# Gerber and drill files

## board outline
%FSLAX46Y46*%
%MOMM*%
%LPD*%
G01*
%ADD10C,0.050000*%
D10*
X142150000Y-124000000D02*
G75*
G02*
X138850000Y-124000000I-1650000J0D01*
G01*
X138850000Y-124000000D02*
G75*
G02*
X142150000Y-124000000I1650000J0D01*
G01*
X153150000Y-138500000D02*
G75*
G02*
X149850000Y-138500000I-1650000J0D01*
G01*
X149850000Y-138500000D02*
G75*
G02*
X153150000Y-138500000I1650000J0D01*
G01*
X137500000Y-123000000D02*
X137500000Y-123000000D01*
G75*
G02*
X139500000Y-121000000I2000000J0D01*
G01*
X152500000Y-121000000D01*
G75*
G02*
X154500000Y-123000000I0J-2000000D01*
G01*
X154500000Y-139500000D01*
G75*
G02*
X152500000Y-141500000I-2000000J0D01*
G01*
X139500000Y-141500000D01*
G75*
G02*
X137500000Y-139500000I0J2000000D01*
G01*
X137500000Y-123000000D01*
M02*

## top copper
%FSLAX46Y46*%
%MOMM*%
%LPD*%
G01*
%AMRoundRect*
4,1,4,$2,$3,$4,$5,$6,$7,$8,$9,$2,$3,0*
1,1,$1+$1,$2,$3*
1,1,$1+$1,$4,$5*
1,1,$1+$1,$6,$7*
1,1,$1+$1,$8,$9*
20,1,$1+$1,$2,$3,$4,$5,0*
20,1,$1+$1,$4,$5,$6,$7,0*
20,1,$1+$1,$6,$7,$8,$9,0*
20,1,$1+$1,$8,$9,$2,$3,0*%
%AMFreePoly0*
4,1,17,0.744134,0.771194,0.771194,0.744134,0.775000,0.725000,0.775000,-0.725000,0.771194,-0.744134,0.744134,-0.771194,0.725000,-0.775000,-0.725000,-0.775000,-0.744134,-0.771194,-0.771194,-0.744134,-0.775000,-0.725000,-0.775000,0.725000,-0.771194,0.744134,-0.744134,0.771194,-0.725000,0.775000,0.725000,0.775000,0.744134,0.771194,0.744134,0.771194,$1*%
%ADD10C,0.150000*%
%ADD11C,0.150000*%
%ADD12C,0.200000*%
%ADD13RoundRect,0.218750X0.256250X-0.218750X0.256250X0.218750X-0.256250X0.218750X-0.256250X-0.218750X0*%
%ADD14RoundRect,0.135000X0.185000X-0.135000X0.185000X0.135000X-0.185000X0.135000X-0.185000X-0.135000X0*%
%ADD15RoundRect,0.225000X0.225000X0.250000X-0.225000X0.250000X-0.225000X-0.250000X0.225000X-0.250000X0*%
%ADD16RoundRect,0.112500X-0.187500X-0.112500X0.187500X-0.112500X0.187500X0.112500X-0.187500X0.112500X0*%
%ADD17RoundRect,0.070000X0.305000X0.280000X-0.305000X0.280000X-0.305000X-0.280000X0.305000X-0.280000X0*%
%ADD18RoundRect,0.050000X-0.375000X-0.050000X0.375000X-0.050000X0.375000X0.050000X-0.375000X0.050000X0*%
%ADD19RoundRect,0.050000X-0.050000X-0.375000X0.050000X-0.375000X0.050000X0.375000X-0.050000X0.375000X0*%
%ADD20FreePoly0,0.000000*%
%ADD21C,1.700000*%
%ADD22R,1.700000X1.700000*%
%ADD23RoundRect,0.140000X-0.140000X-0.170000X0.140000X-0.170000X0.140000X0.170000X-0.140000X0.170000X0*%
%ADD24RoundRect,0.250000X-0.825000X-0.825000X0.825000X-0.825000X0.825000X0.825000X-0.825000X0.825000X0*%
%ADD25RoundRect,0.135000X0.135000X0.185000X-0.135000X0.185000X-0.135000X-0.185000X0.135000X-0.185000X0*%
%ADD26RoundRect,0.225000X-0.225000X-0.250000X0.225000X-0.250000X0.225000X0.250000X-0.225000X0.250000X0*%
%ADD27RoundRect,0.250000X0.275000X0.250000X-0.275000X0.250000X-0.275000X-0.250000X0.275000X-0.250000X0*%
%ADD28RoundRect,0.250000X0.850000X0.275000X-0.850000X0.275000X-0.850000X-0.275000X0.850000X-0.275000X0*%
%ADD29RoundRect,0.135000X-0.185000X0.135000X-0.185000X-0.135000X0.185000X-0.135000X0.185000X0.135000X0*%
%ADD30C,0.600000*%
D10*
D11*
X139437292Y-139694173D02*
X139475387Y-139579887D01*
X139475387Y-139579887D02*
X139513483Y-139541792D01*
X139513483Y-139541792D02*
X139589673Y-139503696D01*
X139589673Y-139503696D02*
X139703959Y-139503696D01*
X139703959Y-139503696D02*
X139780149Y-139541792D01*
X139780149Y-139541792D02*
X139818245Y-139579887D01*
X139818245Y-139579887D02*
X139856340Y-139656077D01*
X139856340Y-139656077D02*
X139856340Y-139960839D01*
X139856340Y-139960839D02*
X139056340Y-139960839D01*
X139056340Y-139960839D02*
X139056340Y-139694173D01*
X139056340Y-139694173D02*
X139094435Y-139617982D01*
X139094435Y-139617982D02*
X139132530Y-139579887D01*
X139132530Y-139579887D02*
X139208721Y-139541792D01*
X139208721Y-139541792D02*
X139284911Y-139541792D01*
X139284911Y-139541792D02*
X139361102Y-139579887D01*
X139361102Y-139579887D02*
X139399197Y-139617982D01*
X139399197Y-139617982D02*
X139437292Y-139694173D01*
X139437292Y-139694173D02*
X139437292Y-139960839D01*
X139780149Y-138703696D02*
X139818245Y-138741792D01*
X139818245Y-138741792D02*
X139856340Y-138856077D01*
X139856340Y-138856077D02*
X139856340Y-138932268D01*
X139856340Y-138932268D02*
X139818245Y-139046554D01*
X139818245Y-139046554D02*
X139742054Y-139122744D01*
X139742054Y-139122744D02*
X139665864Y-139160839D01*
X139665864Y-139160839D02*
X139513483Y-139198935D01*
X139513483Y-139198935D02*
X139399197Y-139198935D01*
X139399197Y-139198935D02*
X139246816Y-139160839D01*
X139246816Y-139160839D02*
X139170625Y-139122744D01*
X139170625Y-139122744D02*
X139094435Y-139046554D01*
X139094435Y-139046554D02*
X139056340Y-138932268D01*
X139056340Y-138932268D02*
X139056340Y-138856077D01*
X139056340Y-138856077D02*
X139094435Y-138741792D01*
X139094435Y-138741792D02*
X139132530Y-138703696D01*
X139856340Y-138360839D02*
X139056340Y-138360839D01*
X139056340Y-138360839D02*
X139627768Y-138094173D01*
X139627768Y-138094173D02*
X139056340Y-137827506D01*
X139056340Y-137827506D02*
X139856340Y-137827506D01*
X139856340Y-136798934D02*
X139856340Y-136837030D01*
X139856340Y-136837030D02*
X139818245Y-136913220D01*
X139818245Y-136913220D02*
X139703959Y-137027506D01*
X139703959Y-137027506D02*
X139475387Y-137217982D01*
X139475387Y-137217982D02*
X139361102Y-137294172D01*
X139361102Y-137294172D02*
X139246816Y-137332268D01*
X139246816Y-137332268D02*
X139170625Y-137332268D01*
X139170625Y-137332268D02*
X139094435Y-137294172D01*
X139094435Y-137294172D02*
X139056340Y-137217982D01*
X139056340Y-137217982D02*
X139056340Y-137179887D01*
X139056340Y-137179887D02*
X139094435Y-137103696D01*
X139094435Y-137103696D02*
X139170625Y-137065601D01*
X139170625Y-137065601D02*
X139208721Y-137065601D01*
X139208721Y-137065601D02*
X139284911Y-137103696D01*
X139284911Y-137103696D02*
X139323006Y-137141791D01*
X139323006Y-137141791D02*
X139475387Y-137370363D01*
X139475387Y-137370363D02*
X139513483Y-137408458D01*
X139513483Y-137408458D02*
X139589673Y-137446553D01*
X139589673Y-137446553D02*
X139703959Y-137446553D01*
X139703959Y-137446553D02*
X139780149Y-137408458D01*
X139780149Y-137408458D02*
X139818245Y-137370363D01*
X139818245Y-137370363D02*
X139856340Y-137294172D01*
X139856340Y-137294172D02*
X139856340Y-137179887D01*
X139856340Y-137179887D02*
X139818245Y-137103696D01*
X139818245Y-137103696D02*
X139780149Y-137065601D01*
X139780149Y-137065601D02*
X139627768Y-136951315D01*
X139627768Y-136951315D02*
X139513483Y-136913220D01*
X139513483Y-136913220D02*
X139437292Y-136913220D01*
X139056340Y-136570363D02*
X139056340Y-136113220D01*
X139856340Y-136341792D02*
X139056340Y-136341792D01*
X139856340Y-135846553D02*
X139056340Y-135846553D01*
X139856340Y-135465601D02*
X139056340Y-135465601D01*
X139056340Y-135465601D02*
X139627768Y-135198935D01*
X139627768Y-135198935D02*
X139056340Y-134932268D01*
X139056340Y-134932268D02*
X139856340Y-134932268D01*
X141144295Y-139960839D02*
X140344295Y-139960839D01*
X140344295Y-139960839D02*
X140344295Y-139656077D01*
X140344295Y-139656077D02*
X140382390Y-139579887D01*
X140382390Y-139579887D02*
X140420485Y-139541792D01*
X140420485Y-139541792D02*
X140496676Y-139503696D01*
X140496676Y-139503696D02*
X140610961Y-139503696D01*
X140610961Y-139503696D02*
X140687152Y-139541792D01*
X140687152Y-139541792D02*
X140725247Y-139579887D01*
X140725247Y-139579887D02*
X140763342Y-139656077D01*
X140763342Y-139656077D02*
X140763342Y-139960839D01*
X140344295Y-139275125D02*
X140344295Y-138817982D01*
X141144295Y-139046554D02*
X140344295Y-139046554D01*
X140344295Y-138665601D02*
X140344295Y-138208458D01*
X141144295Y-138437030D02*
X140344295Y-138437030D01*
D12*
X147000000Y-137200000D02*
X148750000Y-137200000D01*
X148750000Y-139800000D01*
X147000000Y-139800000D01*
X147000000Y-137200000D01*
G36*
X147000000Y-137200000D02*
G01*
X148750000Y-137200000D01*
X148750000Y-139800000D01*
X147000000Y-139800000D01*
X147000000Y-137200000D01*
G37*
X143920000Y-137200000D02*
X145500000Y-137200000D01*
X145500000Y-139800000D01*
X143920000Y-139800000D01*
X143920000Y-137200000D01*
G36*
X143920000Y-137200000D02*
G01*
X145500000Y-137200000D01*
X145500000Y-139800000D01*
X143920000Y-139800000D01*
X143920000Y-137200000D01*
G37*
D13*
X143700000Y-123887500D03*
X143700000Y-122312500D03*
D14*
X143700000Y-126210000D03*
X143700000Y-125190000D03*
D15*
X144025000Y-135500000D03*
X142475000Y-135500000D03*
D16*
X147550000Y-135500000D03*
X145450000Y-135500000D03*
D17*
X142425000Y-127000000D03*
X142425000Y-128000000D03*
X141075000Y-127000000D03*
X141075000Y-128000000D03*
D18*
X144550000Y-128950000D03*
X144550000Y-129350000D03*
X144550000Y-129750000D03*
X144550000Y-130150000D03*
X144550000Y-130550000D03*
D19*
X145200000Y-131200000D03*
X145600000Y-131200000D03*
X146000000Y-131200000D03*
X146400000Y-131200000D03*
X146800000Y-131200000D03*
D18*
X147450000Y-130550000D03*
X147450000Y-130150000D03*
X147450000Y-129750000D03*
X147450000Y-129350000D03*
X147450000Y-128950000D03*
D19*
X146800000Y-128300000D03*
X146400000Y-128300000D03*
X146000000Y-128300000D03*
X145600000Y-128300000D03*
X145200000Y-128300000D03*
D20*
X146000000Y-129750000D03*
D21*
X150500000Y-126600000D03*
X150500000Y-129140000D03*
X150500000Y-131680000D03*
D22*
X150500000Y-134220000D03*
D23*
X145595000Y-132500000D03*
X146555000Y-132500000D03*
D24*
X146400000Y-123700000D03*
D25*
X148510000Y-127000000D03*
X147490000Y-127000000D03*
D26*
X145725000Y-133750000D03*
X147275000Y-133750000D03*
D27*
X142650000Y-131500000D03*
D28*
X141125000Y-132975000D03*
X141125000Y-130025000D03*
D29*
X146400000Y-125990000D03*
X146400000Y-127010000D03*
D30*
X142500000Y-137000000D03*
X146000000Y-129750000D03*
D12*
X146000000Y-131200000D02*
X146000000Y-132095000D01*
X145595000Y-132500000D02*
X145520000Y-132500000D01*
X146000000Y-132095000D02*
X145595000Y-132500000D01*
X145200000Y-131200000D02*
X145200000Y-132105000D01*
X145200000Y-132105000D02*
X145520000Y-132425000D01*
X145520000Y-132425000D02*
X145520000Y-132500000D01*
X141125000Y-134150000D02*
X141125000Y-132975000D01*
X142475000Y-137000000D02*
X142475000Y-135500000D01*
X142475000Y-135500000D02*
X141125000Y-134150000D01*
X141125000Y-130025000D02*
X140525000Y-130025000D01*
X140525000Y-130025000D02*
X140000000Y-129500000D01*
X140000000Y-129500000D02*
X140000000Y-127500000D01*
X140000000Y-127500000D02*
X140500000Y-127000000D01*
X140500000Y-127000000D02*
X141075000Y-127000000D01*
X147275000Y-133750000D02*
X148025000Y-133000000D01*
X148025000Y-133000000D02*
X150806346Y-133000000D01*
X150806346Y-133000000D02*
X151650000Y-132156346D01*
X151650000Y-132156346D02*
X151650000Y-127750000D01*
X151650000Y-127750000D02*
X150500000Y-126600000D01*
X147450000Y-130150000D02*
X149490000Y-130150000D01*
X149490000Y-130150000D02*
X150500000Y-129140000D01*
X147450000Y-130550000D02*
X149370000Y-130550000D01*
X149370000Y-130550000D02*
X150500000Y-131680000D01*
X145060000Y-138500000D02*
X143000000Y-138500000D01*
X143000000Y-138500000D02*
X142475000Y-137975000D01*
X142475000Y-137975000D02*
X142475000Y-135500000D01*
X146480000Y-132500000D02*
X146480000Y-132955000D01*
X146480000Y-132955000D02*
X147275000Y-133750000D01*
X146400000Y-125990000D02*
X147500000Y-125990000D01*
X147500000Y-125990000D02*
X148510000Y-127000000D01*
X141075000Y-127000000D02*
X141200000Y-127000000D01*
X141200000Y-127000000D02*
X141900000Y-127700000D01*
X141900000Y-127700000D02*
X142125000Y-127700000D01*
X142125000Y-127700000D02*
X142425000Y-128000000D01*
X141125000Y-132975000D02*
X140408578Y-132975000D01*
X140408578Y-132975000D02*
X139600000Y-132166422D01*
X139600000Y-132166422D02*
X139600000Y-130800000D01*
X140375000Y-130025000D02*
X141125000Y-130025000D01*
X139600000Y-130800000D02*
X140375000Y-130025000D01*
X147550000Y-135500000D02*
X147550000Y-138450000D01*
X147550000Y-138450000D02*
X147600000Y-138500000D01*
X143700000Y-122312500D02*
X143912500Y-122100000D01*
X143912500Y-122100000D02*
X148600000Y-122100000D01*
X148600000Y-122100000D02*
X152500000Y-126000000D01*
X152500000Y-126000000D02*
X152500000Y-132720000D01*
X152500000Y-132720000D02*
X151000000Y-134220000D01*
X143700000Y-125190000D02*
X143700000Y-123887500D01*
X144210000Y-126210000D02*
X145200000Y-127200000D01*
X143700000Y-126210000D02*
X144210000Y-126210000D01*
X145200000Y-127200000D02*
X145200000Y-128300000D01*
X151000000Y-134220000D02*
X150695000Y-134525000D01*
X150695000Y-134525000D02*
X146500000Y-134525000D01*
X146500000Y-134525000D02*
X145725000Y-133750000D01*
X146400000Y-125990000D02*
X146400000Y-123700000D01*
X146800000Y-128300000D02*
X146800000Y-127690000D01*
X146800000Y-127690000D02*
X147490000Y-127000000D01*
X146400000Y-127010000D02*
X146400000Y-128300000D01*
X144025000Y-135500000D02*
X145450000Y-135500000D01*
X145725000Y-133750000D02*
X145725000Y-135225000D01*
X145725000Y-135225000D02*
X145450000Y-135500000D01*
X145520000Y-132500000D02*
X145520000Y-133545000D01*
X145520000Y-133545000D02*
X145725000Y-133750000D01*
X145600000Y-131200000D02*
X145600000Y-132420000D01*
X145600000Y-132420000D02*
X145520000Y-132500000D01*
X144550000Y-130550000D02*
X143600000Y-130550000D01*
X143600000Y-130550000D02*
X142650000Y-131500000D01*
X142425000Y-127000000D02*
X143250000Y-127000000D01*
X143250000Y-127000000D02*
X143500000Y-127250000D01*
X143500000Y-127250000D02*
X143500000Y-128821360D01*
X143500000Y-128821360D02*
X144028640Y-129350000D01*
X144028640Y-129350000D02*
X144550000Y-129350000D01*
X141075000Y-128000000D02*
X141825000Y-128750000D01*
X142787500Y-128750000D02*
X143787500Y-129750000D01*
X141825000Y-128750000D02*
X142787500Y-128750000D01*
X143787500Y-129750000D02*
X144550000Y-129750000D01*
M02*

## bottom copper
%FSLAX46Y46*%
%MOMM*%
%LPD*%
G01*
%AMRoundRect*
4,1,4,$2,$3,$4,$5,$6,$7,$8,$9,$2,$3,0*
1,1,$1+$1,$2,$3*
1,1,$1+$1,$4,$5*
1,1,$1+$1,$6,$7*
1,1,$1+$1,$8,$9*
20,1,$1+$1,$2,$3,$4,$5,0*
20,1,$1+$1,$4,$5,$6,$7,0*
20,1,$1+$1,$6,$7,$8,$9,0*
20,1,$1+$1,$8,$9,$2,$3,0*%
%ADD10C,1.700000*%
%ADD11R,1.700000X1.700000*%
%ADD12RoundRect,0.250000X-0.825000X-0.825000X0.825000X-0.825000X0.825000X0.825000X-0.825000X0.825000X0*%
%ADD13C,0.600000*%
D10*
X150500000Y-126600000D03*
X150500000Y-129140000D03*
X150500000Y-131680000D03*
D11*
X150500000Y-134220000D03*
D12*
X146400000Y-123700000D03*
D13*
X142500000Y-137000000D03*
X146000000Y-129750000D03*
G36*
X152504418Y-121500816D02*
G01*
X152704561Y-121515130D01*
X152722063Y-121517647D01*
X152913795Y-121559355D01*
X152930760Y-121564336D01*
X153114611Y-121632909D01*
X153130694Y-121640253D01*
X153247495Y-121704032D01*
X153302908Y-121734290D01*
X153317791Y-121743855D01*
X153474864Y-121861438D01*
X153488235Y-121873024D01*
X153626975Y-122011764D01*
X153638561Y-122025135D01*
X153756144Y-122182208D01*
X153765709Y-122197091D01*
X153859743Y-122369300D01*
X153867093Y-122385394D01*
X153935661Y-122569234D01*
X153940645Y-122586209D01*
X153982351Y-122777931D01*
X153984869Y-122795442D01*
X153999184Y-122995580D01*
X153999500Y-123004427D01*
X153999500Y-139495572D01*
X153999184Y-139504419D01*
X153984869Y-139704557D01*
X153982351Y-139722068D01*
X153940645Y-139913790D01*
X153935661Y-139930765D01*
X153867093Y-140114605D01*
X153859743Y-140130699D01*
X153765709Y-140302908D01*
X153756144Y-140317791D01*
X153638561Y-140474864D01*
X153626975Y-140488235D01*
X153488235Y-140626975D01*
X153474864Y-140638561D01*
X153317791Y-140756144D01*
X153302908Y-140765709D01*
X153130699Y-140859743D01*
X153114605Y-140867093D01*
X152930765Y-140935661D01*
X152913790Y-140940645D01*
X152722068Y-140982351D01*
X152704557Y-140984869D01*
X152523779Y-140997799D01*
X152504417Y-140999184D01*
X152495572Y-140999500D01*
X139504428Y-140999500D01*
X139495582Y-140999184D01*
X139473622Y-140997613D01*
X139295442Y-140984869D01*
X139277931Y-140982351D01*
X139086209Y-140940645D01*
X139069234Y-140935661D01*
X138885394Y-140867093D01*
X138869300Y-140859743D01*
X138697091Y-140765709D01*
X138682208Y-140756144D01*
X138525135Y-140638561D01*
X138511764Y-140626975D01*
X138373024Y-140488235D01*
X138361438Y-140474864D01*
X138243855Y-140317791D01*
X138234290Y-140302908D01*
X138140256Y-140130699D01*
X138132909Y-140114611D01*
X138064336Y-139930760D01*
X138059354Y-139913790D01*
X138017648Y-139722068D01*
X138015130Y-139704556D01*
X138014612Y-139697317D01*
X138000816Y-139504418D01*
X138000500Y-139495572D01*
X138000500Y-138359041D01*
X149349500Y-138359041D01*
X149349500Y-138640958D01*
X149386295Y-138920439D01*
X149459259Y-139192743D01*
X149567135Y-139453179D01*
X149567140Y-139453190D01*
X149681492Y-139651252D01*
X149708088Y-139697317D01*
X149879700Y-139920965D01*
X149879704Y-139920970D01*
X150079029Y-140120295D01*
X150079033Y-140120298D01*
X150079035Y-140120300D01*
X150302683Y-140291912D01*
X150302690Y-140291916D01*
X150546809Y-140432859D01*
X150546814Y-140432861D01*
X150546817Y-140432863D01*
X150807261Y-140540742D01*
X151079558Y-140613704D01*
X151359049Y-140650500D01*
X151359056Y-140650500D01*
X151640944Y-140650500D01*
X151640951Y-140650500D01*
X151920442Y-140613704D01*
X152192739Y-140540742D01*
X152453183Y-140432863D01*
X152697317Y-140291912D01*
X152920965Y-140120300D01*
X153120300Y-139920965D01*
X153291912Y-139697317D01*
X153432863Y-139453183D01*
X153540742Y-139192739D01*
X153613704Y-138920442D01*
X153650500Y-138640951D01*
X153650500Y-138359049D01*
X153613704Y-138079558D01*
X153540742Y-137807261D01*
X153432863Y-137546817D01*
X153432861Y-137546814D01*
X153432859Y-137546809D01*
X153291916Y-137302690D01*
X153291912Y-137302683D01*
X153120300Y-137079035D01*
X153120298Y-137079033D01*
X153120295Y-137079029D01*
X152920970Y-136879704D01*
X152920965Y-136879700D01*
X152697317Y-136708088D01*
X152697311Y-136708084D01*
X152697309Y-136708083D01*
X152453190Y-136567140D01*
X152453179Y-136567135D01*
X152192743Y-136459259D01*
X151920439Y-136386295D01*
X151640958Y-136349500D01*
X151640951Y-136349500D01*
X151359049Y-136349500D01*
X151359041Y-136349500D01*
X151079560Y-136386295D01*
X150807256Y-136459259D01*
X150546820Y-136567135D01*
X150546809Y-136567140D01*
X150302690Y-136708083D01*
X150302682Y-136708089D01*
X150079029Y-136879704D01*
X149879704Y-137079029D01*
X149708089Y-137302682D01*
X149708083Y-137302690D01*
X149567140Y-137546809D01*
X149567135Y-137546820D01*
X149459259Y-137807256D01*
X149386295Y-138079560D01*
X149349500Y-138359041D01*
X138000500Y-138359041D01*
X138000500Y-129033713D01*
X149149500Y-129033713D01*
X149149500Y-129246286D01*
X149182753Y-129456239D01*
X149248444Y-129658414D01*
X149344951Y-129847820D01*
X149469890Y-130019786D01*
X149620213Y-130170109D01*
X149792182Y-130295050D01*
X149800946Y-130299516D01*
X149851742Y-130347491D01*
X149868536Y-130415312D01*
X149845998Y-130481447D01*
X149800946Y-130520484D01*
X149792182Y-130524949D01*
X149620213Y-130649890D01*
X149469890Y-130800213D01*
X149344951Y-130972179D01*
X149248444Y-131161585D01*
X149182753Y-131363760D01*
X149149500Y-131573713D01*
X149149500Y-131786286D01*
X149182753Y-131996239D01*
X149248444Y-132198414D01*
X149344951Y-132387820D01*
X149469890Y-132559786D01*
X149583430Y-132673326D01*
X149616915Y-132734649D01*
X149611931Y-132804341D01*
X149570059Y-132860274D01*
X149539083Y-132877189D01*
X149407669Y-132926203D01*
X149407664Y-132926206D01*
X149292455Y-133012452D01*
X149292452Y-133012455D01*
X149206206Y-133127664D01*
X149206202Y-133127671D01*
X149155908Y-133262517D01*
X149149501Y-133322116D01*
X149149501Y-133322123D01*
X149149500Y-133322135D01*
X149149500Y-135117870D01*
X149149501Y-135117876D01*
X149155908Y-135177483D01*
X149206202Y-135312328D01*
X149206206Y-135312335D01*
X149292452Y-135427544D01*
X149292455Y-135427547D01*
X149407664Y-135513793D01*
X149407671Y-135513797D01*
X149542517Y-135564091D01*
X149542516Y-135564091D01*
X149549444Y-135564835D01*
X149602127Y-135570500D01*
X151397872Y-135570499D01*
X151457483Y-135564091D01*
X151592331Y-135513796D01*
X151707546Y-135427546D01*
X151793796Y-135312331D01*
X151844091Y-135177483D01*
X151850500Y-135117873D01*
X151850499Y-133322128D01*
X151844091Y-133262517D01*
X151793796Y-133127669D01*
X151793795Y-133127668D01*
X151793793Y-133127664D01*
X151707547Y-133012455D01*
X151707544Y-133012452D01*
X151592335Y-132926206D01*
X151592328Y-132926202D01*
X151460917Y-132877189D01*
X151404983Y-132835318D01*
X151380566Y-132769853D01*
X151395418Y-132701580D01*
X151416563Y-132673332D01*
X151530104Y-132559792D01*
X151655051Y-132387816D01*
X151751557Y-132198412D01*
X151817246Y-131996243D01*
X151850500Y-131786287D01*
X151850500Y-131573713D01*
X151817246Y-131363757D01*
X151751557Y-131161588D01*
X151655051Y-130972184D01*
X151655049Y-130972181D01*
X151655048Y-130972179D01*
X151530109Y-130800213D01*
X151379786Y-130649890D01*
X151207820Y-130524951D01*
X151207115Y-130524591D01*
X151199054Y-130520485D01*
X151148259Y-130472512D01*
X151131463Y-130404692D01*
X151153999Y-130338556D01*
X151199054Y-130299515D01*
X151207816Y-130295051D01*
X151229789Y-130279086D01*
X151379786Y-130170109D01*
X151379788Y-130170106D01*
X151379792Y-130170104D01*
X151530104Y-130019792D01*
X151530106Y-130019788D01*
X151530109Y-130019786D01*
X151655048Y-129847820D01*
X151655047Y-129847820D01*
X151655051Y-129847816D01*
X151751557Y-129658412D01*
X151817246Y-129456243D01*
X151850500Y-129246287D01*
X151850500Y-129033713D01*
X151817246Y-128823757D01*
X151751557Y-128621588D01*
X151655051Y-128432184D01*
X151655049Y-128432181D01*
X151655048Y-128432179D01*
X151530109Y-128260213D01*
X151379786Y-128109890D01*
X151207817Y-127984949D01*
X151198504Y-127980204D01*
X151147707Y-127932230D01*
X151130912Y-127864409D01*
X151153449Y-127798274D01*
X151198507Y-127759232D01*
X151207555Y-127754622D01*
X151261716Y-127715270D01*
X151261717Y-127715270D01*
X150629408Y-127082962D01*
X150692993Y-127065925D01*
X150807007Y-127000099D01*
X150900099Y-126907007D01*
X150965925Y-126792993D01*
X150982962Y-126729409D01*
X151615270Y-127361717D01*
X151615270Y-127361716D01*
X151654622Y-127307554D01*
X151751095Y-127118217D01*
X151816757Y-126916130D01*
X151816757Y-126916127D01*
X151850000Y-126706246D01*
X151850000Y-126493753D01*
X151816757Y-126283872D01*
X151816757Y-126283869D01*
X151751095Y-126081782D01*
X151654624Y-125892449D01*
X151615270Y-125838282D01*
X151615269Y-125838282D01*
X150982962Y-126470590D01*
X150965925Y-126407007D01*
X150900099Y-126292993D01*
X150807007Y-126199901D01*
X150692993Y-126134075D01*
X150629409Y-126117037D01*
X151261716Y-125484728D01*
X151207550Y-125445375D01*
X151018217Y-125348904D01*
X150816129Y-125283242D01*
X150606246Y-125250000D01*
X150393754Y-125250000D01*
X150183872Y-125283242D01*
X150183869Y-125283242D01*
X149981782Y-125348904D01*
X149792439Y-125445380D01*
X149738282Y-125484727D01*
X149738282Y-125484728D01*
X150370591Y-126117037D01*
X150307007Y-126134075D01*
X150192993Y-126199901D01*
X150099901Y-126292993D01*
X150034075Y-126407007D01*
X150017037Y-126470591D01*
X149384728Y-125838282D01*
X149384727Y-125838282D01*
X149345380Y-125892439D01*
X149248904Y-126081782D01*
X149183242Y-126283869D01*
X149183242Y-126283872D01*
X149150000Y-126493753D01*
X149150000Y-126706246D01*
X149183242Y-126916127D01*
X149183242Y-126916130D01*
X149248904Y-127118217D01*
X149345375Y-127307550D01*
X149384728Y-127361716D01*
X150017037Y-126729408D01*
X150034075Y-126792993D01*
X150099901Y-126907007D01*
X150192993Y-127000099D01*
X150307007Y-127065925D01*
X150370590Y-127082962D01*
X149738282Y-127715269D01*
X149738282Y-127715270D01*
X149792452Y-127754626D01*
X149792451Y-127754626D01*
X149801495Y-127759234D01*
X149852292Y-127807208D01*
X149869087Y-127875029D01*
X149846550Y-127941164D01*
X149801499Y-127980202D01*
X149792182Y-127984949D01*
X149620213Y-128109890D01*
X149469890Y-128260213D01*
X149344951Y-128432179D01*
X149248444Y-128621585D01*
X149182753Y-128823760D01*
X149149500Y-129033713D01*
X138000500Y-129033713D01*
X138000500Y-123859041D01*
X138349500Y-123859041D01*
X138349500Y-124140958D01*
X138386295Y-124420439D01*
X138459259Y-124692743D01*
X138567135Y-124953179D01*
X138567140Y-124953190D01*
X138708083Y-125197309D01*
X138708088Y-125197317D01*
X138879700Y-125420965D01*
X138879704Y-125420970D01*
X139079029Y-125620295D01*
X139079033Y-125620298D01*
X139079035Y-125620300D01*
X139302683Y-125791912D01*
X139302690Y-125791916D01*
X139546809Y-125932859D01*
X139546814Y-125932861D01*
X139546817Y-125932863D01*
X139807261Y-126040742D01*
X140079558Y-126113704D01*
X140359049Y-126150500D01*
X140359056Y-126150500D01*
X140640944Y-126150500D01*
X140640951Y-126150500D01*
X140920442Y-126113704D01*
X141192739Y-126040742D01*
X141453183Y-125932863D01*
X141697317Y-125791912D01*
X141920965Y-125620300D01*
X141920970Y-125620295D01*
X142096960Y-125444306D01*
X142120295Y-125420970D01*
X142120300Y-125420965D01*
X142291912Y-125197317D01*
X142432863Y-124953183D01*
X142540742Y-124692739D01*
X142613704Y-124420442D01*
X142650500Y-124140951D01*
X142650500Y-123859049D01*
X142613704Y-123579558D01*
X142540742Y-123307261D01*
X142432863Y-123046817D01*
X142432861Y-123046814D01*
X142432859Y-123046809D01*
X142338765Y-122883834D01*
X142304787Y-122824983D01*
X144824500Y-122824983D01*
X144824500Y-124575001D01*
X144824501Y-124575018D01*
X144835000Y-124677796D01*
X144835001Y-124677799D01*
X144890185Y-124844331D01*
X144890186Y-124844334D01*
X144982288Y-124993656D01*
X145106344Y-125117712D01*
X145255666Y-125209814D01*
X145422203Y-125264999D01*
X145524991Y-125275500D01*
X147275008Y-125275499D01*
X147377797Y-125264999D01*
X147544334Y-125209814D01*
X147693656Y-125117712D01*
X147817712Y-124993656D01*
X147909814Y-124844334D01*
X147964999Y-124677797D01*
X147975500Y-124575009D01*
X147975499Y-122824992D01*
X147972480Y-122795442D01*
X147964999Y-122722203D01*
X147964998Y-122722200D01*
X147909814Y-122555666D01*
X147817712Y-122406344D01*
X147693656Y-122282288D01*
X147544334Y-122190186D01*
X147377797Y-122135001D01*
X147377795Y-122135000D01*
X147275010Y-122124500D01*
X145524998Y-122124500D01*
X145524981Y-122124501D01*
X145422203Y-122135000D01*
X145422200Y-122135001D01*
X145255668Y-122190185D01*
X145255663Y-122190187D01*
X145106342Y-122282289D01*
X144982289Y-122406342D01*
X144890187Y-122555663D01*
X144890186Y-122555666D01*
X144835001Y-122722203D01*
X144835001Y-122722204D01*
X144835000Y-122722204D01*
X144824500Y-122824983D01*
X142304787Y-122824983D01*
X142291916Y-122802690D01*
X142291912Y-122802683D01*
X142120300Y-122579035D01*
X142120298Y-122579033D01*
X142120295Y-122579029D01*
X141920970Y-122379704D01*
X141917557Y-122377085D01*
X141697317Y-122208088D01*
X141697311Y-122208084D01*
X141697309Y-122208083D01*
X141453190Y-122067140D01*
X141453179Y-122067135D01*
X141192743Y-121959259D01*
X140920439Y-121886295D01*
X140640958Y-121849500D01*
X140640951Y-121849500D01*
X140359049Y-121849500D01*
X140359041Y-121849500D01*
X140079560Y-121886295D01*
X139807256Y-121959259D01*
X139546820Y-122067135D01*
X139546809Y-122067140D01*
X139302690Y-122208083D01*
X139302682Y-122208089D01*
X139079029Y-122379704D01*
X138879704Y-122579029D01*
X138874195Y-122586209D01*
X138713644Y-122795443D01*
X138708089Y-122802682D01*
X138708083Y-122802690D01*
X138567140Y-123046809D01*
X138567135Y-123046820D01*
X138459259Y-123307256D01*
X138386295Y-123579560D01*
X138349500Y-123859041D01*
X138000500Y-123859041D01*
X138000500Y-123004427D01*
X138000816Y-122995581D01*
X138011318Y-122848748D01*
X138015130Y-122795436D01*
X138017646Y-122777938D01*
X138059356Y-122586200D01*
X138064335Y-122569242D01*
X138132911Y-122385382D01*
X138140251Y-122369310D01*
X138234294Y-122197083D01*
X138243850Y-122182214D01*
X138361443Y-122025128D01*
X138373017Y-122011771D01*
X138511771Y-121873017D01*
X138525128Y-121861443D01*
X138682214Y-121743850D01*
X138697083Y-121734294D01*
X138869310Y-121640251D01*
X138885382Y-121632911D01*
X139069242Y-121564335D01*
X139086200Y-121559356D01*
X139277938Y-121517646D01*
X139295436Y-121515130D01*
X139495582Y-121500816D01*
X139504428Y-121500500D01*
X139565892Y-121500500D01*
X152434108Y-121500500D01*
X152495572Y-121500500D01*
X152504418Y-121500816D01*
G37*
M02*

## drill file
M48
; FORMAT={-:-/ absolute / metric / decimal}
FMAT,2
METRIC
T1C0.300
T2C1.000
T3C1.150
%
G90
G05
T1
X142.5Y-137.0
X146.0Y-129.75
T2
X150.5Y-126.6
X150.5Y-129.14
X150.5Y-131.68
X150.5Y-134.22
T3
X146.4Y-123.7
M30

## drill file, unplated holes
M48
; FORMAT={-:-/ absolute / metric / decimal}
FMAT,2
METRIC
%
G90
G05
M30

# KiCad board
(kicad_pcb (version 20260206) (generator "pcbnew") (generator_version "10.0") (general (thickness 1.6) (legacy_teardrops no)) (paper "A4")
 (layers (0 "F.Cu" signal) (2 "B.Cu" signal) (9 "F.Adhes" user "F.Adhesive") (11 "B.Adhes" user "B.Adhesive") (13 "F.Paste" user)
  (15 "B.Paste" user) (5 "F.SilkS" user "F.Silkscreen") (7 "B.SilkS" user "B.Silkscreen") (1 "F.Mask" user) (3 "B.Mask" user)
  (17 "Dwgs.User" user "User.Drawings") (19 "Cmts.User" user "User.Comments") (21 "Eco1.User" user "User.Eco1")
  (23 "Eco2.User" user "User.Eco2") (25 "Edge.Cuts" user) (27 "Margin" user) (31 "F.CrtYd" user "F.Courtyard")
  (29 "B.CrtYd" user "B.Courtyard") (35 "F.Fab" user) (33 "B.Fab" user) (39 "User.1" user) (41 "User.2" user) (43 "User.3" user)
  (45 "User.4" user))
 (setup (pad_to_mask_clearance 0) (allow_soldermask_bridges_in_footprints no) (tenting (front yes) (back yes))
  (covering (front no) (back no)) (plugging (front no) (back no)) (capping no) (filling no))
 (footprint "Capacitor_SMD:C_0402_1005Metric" (layer "F.Cu") (at 146.075 132.5)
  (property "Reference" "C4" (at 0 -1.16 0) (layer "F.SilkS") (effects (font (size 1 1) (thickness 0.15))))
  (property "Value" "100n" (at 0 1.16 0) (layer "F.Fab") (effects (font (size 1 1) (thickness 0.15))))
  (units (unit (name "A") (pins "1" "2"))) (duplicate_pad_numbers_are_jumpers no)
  (pad "1" smd roundrect (at -0.48 0) (size 0.56 0.62) (layers "F.Cu" "F.Mask" "F.Paste") (roundrect_rratio 0.25) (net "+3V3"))
  (pad "2" smd roundrect (at 0.48 0) (size 0.56 0.62) (layers "F.Cu" "F.Mask" "F.Paste") (roundrect_rratio 0.25) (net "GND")))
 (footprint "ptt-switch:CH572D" (layer "F.Cu") (at 146 129.75)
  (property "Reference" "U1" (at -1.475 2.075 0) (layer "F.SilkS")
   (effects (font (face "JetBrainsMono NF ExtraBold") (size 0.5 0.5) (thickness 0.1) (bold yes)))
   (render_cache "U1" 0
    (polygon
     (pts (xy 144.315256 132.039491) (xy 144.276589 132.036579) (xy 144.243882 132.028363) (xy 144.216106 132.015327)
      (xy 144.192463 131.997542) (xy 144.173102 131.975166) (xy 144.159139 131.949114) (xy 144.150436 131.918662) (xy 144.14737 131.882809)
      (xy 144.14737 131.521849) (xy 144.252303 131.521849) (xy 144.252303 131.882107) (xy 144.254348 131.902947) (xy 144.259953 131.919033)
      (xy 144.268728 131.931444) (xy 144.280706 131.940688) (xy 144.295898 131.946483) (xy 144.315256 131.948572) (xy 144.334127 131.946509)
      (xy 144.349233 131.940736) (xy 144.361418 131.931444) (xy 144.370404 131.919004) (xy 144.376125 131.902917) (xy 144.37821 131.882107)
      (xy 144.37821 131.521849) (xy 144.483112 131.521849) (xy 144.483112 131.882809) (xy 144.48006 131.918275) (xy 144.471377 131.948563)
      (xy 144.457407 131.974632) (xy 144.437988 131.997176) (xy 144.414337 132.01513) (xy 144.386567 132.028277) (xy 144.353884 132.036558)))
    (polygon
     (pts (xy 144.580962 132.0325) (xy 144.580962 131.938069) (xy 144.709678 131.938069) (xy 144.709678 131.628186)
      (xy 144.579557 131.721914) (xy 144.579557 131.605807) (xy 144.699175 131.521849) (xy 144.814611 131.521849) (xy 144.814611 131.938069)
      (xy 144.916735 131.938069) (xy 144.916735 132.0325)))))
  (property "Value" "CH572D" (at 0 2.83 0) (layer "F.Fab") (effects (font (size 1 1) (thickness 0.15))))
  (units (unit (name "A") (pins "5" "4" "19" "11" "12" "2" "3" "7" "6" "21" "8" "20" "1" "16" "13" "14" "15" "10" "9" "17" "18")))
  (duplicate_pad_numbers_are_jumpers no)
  (pad "" smd roundrect (at -0.45 -0.45) (size 0.4 0.4) (layers "F.Paste") (roundrect_rratio 0.25))
  (pad "" smd roundrect (at -0.45 0.45) (size 0.4 0.4) (layers "F.Paste") (roundrect_rratio 0.25))
  (pad "" smd roundrect (at 0.45 -0.45) (size 0.4 0.4) (layers "F.Paste") (roundrect_rratio 0.25))
  (pad "" smd roundrect (at 0.45 0.45) (size 0.4 0.4) (layers "F.Paste") (roundrect_rratio 0.25))
  (pad "1" smd roundrect (at -1.45 -0.8) (size 0.85 0.2) (layers "F.Cu" "F.Mask" "F.Paste") (roundrect_rratio 0.25)
   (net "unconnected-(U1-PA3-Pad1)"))
  (pad "2" smd roundrect (at -1.45 -0.4) (size 0.85 0.2) (layers "F.Cu" "F.Mask" "F.Paste") (roundrect_rratio 0.25) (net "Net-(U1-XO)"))
  (pad "3" smd roundrect (at -1.45 0) (size 0.85 0.2) (layers "F.Cu" "F.Mask" "F.Paste") (roundrect_rratio 0.25) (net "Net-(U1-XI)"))
  (pad "4" smd roundrect (at -1.45 0.4) (size 0.85 0.2) (layers "F.Cu" "F.Mask" "F.Paste") (roundrect_rratio 0.25)
   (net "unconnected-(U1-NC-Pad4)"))
  (pad "5" smd roundrect (at -1.45 0.8) (size 0.85 0.2) (layers "F.Cu" "F.Mask" "F.Paste") (roundrect_rratio 0.25) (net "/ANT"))
  (pad "6" smd roundrect (at -0.8 1.45) (size 0.2 0.85) (layers "F.Cu" "F.Mask" "F.Paste") (roundrect_rratio 0.25) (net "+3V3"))
  (pad "7" smd roundrect (at -0.4 1.45) (size 0.2 0.85) (layers "F.Cu" "F.Mask" "F.Paste") (roundrect_rratio 0.25) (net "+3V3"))
  (pad "8" smd roundrect (at 0 1.45) (size 0.2 0.85) (layers "F.Cu" "F.Mask" "F.Paste") (roundrect_rratio 0.25) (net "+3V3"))
  (pad "9" smd roundrect (at 0.4 1.45) (size 0.2 0.85) (layers "F.Cu" "F.Mask" "F.Paste") (roundrect_rratio 0.25)
   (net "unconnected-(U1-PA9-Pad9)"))
  (pad "10" smd roundrect (at 0.8 1.45) (size 0.2 0.85) (layers "F.Cu" "F.Mask" "F.Paste") (roundrect_rratio 0.25)
   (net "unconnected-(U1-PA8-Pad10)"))
  (pad "11" smd roundrect (at 1.45 0.8) (size 0.85 0.2) (layers "F.Cu" "F.Mask" "F.Paste") (roundrect_rratio 0.25) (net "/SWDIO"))
  (pad "12" smd roundrect (at 1.45 0.4) (size 0.85 0.2) (layers "F.Cu" "F.Mask" "F.Paste") (roundrect_rratio 0.25) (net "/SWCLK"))
  (pad "13" smd roundrect (at 1.45 0) (size 0.85 0.2) (layers "F.Cu" "F.Mask" "F.Paste") (roundrect_rratio 0.25)
   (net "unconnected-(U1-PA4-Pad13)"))
  (pad "14" smd roundrect (at 1.45 -0.4) (size 0.85 0.2) (layers "F.Cu" "F.Mask" "F.Paste") (roundrect_rratio 0.25)
   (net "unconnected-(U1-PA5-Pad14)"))
  (pad "15" smd roundrect (at 1.45 -0.8) (size 0.85 0.2) (layers "F.Cu" "F.Mask" "F.Paste") (roundrect_rratio 0.25)
   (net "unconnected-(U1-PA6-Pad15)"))
  (pad "16" smd roundrect (at 0.8 -1.45) (size 0.2 0.85) (layers "F.Cu" "F.Mask" "F.Paste") (roundrect_rratio 0.25) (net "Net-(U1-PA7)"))
  (pad "17" smd roundrect (at 0.4 -1.45) (size 0.2 0.85) (layers "F.Cu" "F.Mask" "F.Paste") (roundrect_rratio 0.25) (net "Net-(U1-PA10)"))
  (pad "18" smd roundrect (at 0 -1.45) (size 0.2 0.85) (layers "F.Cu" "F.Mask" "F.Paste") (roundrect_rratio 0.25)
   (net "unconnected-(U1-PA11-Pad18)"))
  (pad "19" smd roundrect (at -0.4 -1.45) (size 0.2 0.85) (layers "F.Cu" "F.Mask" "F.Paste") (roundrect_rratio 0.25)
   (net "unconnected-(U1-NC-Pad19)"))
  (pad "20" smd roundrect (at -0.8 -1.45) (size 0.2 0.85) (layers "F.Cu" "F.Mask" "F.Paste") (roundrect_rratio 0.25) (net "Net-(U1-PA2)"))
  (pad "21" smd custom (at 0 0) (size 1.45 1.45) (layers "F.Cu") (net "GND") (thermal_bridge_angle 90)
   (options (clearance outline) (anchor circle)) (primitives)))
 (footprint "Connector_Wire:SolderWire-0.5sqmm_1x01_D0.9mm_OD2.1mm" (layer "F.Cu") (at 146.4 123.7)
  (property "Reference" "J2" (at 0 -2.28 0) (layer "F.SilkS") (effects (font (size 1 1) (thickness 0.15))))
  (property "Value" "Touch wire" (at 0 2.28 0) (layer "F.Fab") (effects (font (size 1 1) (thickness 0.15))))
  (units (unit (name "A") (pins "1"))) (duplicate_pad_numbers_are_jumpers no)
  (pad "1" thru_hole roundrect (at 0 0) (size 2.15 2.15) (drill 1.15) (layers "*.Cu" "*.Mask") (remove_unused_layers no)
   (roundrect_rratio 0.116279) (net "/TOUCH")))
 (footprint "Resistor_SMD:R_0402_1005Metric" (layer "F.Cu") (at 148 127 180)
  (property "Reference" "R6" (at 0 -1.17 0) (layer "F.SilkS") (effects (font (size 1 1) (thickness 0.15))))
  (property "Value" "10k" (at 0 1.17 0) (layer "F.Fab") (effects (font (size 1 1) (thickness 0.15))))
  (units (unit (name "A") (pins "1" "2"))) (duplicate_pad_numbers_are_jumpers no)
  (pad "1" smd roundrect (at -0.51 0 180) (size 0.54 0.64) (layers "F.Cu" "F.Mask" "F.Paste") (roundrect_rratio 0.25) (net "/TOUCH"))
  (pad "2" smd roundrect (at 0.51 0 180) (size 0.54 0.64) (layers "F.Cu" "F.Mask" "F.Paste") (roundrect_rratio 0.25) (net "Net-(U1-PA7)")))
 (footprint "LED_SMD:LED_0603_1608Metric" (layer "F.Cu") (at 143.7 123.1 90)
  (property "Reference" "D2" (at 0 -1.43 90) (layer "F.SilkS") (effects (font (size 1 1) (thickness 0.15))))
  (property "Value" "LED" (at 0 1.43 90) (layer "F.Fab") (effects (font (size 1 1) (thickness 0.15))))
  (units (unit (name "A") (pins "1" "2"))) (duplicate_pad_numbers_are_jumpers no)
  (pad "1" smd roundrect (at -0.7875 0 90) (size 0.875 0.95) (layers "F.Cu" "F.Mask" "F.Paste") (roundrect_rratio 0.25) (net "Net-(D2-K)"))
  (pad "2" smd roundrect (at 0.7875 0 90) (size 0.875 0.95) (layers "F.Cu" "F.Mask" "F.Paste") (roundrect_rratio 0.25) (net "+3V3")))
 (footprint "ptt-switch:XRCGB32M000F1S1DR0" (layer "F.Cu") (at 141.75 127.5 180)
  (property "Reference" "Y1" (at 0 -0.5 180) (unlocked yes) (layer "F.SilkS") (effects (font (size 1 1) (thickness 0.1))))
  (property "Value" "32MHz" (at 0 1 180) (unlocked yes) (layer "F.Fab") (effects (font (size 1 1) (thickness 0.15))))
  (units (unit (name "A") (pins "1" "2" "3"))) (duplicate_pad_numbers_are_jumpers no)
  (pad "1" smd roundrect (at -0.675 0.5 180) (size 0.75 0.7) (layers "F.Cu" "F.Mask" "F.Paste") (roundrect_rratio 0.1) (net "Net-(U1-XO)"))
  (pad "2" smd roundrect (at -0.675 -0.5 180) (size 0.75 0.7) (layers "F.Cu" "F.Mask" "F.Paste") (roundrect_rratio 0.1) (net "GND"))
  (pad "2" smd roundrect (at 0.675 0.5 180) (size 0.75 0.7) (layers "F.Cu" "F.Mask" "F.Paste") (roundrect_rratio 0.1) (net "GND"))
  (pad "3" smd roundrect (at 0.675 -0.5 180) (size 0.75 0.7) (layers "F.Cu" "F.Mask" "F.Paste") (roundrect_rratio 0.1) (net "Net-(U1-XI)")))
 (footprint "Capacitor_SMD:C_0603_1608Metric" (layer "F.Cu") (at 146.5 133.75)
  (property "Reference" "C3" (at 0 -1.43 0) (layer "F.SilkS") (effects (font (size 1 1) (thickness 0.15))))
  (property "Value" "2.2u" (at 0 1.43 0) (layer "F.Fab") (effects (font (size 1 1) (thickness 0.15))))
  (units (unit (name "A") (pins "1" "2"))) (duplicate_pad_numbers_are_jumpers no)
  (pad "1" smd roundrect (at -0.775 0) (size 0.9 0.95) (layers "F.Cu" "F.Mask" "F.Paste") (roundrect_rratio 0.25) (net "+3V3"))
  (pad "2" smd roundrect (at 0.775 0) (size 0.9 0.95) (layers "F.Cu" "F.Mask" "F.Paste") (roundrect_rratio 0.25) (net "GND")))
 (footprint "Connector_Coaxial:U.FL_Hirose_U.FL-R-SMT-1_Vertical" (layer "F.Cu") (at 141.125 131.5 180)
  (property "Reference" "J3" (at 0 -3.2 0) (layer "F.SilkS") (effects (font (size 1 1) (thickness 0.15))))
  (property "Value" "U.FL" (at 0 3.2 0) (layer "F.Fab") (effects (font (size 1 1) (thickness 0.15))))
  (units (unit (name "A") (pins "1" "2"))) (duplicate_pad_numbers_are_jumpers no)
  (pad "1" smd roundrect (at -1.525 0 180) (size 1.05 1) (layers "F.Cu" "F.Mask" "F.Paste") (roundrect_rratio 0.25) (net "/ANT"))
  (pad "2" smd roundrect (at 0 -1.475 180) (size 2.2 1.05) (layers "F.Cu" "F.Mask" "F.Paste") (roundrect_rratio 0.2380952381) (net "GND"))
  (pad "2" smd roundrect (at 0 1.475 180) (size 2.2 1.05) (layers "F.Cu" "F.Mask" "F.Paste") (roundrect_rratio 0.2380952381) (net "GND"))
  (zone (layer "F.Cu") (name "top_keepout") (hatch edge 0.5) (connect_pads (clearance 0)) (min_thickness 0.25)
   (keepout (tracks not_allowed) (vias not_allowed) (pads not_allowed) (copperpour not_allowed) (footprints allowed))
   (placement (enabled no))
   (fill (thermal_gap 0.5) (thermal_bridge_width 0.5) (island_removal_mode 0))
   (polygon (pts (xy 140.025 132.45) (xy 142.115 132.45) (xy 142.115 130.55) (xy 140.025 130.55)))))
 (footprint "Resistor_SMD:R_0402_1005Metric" (layer "F.Cu") (at 146.4 126.5 -90)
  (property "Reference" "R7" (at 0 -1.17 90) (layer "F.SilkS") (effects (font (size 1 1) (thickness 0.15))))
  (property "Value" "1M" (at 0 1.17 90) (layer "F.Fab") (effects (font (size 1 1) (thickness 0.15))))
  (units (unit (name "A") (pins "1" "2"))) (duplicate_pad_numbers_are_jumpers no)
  (pad "1" smd roundrect (at -0.51 0 270) (size 0.54 0.64) (layers "F.Cu" "F.Mask" "F.Paste") (roundrect_rratio 0.25) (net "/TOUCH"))
  (pad "2" smd roundrect (at 0.51 0 270) (size 0.54 0.64) (layers "F.Cu" "F.Mask" "F.Paste") (roundrect_rratio 0.25) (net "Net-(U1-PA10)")))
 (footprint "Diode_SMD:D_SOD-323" (layer "F.Cu") (at 146.5 135.5)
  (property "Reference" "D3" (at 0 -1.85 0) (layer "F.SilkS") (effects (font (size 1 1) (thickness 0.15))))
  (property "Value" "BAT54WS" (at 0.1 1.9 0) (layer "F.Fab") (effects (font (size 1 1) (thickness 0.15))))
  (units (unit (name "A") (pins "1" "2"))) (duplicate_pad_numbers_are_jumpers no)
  (pad "1" smd roundrect (at -1.05 0) (size 0.6 0.45) (layers "F.Cu" "F.Mask" "F.Paste") (roundrect_rratio 0.25) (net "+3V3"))
  (pad "2" smd roundrect (at 1.05 0) (size 0.6 0.45) (layers "F.Cu" "F.Mask" "F.Paste") (roundrect_rratio 0.25) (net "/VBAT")))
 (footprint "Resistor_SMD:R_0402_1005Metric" (layer "F.Cu") (at 143.7 125.7 90)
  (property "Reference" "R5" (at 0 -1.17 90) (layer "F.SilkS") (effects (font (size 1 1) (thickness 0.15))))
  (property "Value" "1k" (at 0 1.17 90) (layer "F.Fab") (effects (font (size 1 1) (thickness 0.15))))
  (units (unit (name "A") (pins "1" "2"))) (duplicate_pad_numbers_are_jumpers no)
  (pad "1" smd roundrect (at -0.51 0 90) (size 0.54 0.64) (layers "F.Cu" "F.Mask" "F.Paste") (roundrect_rratio 0.25) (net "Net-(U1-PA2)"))
  (pad "2" smd roundrect (at 0.51 0 90) (size 0.54 0.64) (layers "F.Cu" "F.Mask" "F.Paste") (roundrect_rratio 0.25) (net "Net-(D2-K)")))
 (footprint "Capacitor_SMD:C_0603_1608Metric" (layer "F.Cu") (at 143.25 135.5 180)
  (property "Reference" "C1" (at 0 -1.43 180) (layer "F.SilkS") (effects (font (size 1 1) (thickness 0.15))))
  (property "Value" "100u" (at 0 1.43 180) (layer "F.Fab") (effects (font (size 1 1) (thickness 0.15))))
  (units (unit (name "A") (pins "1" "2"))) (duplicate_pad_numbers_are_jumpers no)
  (pad "1" smd roundrect (at -0.775 0 180) (size 0.9 0.95) (layers "F.Cu" "F.Mask" "F.Paste") (roundrect_rratio 0.25) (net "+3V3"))
  (pad "2" smd roundrect (at 0.775 0 180) (size 0.9 0.95) (layers "F.Cu" "F.Mask" "F.Paste") (roundrect_rratio 0.25) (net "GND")))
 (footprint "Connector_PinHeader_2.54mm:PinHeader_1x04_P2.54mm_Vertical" (layer "F.Cu") (at 150.5 134.22 180)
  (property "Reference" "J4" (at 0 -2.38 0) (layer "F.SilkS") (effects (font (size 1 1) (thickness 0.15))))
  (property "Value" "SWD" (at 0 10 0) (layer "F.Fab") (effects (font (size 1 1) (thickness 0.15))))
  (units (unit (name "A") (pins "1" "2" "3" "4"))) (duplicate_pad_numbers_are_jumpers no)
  (pad "1" thru_hole rect (at 0 0 180) (size 1.7 1.7) (drill 1) (layers "*.Cu" "*.Mask") (remove_unused_layers no) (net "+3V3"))
  (pad "2" thru_hole circle (at 0 2.54 180) (size 1.7 1.7) (drill 1) (layers "*.Cu" "*.Mask") (remove_unused_layers no) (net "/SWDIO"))
  (pad "3" thru_hole circle (at 0 5.08 180) (size 1.7 1.7) (drill 1) (layers "*.Cu" "*.Mask") (remove_unused_layers no) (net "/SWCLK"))
  (pad "4" thru_hole circle (at 0 7.62 180) (size 1.7 1.7) (drill 1) (layers "*.Cu" "*.Mask") (remove_unused_layers no) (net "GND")))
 (gr_rect (start 143.92 137.2) (end 145.5 139.8) (stroke (width 0.2) (type solid)) (fill yes) (layer "F.Cu") (net "GND"))
 (gr_rect (start 147 137.2) (end 148.75 139.8) (stroke (width 0.2) (type solid)) (fill yes) (layer "F.Cu") (net "/VBAT"))
 (gr_rect (start 137.5 121) (end 154.5 141.5) (radius 2) (stroke (width 0.05) (type solid)) (fill no) (layer "Edge.Cuts"))
 (gr_circle (center 140.5 124) (end 142.15 124) (stroke (width 0.05) (type solid)) (fill no) (layer "Edge.Cuts"))
 (gr_circle (center 151.5 138.5) (end 153.15 138.5) (stroke (width 0.05) (type solid)) (fill no) (layer "Edge.Cuts"))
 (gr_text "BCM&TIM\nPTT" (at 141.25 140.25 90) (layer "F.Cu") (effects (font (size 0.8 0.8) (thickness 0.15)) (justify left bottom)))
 (segment (start 145.725 135.225) (end 145.45 135.5) (width 0.2) (layer "F.Cu") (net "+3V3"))
 (segment (start 145.6 131.2) (end 145.6 132.42) (width 0.2) (layer "F.Cu") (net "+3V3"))
 (segment (start 152.5 126) (end 152.5 132.72) (width 0.2) (layer "F.Cu") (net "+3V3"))
 (segment (start 152.5 132.72) (end 151 134.22) (width 0.2) (layer "F.Cu") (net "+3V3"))
 (segment (start 145.2 131.2) (end 145.2 132.105) (width 0.2) (layer "F.Cu") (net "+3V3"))
 (segment (start 143.7 122.3125) (end 143.9125 122.1) (width 0.2) (layer "F.Cu") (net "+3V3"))
 (segment (start 145.52 133.545) (end 145.725 133.75) (width 0.2) (layer "F.Cu") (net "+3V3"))
 (segment (start 151 134.22) (end 150.695 134.525) (width 0.2) (layer "F.Cu") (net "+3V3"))
 (segment (start 146.5 134.525) (end 145.725 133.75) (width 0.2) (layer "F.Cu") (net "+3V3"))
 (segment (start 146 131.2) (end 146 132.095) (width 0.2) (layer "F.Cu") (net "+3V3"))
 (segment (start 144.025 135.5) (end 145.45 135.5) (width 0.2) (layer "F.Cu") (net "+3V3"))
 (segment (start 145.6 132.42) (end 145.52 132.5) (width 0.2) (layer "F.Cu") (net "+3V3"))
 (segment (start 145.595 132.5) (end 145.52 132.5) (width 0.2) (layer "F.Cu") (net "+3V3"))
 (segment (start 145.2 132.105) (end 145.52 132.425) (width 0.2) (layer "F.Cu") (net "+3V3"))
 (segment (start 146 132.095) (end 145.595 132.5) (width 0.2) (layer "F.Cu") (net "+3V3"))
 (segment (start 150.695 134.525) (end 146.5 134.525) (width 0.2) (layer "F.Cu") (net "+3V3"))
 (segment (start 143.9125 122.1) (end 148.6 122.1) (width 0.2) (layer "F.Cu") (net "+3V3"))
 (segment (start 145.725 133.75) (end 145.725 135.225) (width 0.2) (layer "F.Cu") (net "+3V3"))
 (segment (start 148.6 122.1) (end 152.5 126) (width 0.2) (layer "F.Cu") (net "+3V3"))
 (segment (start 145.52 132.5) (end 145.52 133.545) (width 0.2) (layer "F.Cu") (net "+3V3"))
 (segment (start 145.52 132.425) (end 145.52 132.5) (width 0.2) (layer "F.Cu") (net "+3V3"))
 (segment (start 141.125 132.975) (end 140.408578 132.975) (width 0.2) (layer "F.Cu") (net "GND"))
 (segment (start 140.408578 132.975) (end 139.6 132.166422) (width 0.2) (layer "F.Cu") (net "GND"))
 (segment (start 147.275 133.75) (end 148.025 133) (width 0.2) (layer "F.Cu") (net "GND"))
 (segment (start 141.9 127.7) (end 142.125 127.7) (width 0.2) (layer "F.Cu") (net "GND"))
 (segment (start 146.48 132.955) (end 147.275 133.75) (width 0.2) (layer "F.Cu") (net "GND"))
 (segment (start 142.125 127.7) (end 142.425 128) (width 0.2) (layer "F.Cu") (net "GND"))
 (segment (start 140 129.5) (end 140 127.5) (width 0.2) (layer "F.Cu") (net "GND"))
 (segment (start 141.2 127) (end 141.9 127.7) (width 0.2) (layer "F.Cu") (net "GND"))
 (segment (start 150.806346 133) (end 151.65 132.156346) (width 0.2) (layer "F.Cu") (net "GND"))
 (segment (start 141.125 130.025) (end 140.525 130.025) (width 0.2) (layer "F.Cu") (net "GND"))
 (segment (start 139.6 132.166422) (end 139.6 130.8) (width 0.2) (layer "F.Cu") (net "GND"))
 (segment (start 140.525 130.025) (end 140 129.5) (width 0.2) (layer "F.Cu") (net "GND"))
 (segment (start 142.475 137) (end 142.475 135.5) (width 0.2) (layer "F.Cu") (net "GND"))
 (segment (start 141.125 134.15) (end 141.125 132.975) (width 0.2) (layer "F.Cu") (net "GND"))
 (segment (start 151.65 132.156346) (end 151.65 127.75) (width 0.2) (layer "F.Cu") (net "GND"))
 (segment (start 141.075 127) (end 141.2 127) (width 0.2) (layer "F.Cu") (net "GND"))
 (segment (start 140.375 130.025) (end 141.125 130.025) (width 0.2) (layer "F.Cu") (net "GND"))
 (segment (start 145.06 138.5) (end 143 138.5) (width 0.2) (layer "F.Cu") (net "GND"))
 (segment (start 139.6 130.8) (end 140.375 130.025) (width 0.2) (layer "F.Cu") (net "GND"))
 (segment (start 148.025 133) (end 150.806346 133) (width 0.2) (layer "F.Cu") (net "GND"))
 (segment (start 140.5 127) (end 141.075 127) (width 0.2) (layer "F.Cu") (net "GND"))
 (segment (start 151.65 127.75) (end 150.5 126.6) (width 0.2) (layer "F.Cu") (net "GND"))
 (segment (start 143 138.5) (end 142.475 137.975) (width 0.2) (layer "F.Cu") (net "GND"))
 (segment (start 146.48 132.5) (end 146.48 132.955) (width 0.2) (layer "F.Cu") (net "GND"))
 (segment (start 142.475 137.975) (end 142.475 135.5) (width 0.2) (layer "F.Cu") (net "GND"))
 (segment (start 140 127.5) (end 140.5 127) (width 0.2) (layer "F.Cu") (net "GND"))
 (segment (start 142.475 135.5) (end 141.125 134.15) (width 0.2) (layer "F.Cu") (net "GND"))
 (via (at 142.5 137) (size 0.6) (drill 0.3) (layers "F.Cu" "B.Cu") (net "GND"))
 (via (at 146 129.75) (size 0.6) (drill 0.3) (layers "F.Cu" "B.Cu") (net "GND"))
 (segment (start 144.55 130.55) (end 143.6 130.55) (width 0.2) (layer "F.Cu") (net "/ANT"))
 (segment (start 143.6 130.55) (end 142.65 131.5) (width 0.2) (layer "F.Cu") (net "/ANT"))
 (segment (start 147.5 125.99) (end 148.51 127) (width 0.2) (layer "F.Cu") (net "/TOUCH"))
 (segment (start 146.4 125.99) (end 147.5 125.99) (width 0.2) (layer "F.Cu") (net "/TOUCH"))
 (segment (start 146.4 125.99) (end 146.4 123.7) (width 0.2) (layer "F.Cu") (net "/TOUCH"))
 (segment (start 146.8 128.3) (end 146.8 127.69) (width 0.2) (layer "F.Cu") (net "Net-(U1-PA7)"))
 (segment (start 146.8 127.69) (end 147.49 127) (width 0.2) (layer "F.Cu") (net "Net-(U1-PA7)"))
 (segment (start 143.7 125.19) (end 143.7 123.8875) (width 0.2) (layer "F.Cu") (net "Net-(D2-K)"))
 (segment (start 146.4 127.01) (end 146.4 128.3) (width 0.2) (layer "F.Cu") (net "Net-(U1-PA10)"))
 (segment (start 145.2 127.2) (end 145.2 128.3) (width 0.2) (layer "F.Cu") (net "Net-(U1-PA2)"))
 (segment (start 144.21 126.21) (end 145.2 127.2) (width 0.2) (layer "F.Cu") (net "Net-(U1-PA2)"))
 (segment (start 143.7 126.21) (end 144.21 126.21) (width 0.2) (layer "F.Cu") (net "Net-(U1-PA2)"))
 (segment (start 147.55 138.45) (end 147.6 138.5) (width 0.2) (layer "F.Cu") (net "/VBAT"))
 (segment (start 147.55 135.5) (end 147.55 138.45) (width 0.2) (layer "F.Cu") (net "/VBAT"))
 (segment (start 149.37 130.55) (end 150.5 131.68) (width 0.2) (layer "F.Cu") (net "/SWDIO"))
 (segment (start 147.45 130.55) (end 149.37 130.55) (width 0.2) (layer "F.Cu") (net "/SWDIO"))
 (segment (start 147.45 130.15) (end 149.49 130.15) (width 0.2) (layer "F.Cu") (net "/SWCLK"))
 (segment (start 149.49 130.15) (end 150.5 129.14) (width 0.2) (layer "F.Cu") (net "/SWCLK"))
 (segment (start 143.7875 129.75) (end 144.55 129.75) (width 0.2) (layer "F.Cu") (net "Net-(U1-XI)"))
 (segment (start 141.825 128.75) (end 142.7875 128.75) (width 0.2) (layer "F.Cu") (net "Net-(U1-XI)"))
 (segment (start 142.7875 128.75) (end 143.7875 129.75) (width 0.2) (layer "F.Cu") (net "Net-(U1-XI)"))
 (segment (start 141.075 128) (end 141.825 128.75) (width 0.2) (layer "F.Cu") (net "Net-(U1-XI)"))
 (segment (start 144.02864 129.35) (end 144.55 129.35) (width 0.2) (layer "F.Cu") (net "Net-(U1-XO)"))
 (segment (start 142.425 127) (end 143.25 127) (width 0.2) (layer "F.Cu") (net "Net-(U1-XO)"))
 (segment (start 143.25 127) (end 143.5 127.25) (width 0.2) (layer "F.Cu") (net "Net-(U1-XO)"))
 (segment (start 143.5 127.25) (end 143.5 128.82136) (width 0.2) (layer "F.Cu") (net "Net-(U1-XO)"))
 (segment (start 143.5 128.82136) (end 144.02864 129.35) (width 0.2) (layer "F.Cu") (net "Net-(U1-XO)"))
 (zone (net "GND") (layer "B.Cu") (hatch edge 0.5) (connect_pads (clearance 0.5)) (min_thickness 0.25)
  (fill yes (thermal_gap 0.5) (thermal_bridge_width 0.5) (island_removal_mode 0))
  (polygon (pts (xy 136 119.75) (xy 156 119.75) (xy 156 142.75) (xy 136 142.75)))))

